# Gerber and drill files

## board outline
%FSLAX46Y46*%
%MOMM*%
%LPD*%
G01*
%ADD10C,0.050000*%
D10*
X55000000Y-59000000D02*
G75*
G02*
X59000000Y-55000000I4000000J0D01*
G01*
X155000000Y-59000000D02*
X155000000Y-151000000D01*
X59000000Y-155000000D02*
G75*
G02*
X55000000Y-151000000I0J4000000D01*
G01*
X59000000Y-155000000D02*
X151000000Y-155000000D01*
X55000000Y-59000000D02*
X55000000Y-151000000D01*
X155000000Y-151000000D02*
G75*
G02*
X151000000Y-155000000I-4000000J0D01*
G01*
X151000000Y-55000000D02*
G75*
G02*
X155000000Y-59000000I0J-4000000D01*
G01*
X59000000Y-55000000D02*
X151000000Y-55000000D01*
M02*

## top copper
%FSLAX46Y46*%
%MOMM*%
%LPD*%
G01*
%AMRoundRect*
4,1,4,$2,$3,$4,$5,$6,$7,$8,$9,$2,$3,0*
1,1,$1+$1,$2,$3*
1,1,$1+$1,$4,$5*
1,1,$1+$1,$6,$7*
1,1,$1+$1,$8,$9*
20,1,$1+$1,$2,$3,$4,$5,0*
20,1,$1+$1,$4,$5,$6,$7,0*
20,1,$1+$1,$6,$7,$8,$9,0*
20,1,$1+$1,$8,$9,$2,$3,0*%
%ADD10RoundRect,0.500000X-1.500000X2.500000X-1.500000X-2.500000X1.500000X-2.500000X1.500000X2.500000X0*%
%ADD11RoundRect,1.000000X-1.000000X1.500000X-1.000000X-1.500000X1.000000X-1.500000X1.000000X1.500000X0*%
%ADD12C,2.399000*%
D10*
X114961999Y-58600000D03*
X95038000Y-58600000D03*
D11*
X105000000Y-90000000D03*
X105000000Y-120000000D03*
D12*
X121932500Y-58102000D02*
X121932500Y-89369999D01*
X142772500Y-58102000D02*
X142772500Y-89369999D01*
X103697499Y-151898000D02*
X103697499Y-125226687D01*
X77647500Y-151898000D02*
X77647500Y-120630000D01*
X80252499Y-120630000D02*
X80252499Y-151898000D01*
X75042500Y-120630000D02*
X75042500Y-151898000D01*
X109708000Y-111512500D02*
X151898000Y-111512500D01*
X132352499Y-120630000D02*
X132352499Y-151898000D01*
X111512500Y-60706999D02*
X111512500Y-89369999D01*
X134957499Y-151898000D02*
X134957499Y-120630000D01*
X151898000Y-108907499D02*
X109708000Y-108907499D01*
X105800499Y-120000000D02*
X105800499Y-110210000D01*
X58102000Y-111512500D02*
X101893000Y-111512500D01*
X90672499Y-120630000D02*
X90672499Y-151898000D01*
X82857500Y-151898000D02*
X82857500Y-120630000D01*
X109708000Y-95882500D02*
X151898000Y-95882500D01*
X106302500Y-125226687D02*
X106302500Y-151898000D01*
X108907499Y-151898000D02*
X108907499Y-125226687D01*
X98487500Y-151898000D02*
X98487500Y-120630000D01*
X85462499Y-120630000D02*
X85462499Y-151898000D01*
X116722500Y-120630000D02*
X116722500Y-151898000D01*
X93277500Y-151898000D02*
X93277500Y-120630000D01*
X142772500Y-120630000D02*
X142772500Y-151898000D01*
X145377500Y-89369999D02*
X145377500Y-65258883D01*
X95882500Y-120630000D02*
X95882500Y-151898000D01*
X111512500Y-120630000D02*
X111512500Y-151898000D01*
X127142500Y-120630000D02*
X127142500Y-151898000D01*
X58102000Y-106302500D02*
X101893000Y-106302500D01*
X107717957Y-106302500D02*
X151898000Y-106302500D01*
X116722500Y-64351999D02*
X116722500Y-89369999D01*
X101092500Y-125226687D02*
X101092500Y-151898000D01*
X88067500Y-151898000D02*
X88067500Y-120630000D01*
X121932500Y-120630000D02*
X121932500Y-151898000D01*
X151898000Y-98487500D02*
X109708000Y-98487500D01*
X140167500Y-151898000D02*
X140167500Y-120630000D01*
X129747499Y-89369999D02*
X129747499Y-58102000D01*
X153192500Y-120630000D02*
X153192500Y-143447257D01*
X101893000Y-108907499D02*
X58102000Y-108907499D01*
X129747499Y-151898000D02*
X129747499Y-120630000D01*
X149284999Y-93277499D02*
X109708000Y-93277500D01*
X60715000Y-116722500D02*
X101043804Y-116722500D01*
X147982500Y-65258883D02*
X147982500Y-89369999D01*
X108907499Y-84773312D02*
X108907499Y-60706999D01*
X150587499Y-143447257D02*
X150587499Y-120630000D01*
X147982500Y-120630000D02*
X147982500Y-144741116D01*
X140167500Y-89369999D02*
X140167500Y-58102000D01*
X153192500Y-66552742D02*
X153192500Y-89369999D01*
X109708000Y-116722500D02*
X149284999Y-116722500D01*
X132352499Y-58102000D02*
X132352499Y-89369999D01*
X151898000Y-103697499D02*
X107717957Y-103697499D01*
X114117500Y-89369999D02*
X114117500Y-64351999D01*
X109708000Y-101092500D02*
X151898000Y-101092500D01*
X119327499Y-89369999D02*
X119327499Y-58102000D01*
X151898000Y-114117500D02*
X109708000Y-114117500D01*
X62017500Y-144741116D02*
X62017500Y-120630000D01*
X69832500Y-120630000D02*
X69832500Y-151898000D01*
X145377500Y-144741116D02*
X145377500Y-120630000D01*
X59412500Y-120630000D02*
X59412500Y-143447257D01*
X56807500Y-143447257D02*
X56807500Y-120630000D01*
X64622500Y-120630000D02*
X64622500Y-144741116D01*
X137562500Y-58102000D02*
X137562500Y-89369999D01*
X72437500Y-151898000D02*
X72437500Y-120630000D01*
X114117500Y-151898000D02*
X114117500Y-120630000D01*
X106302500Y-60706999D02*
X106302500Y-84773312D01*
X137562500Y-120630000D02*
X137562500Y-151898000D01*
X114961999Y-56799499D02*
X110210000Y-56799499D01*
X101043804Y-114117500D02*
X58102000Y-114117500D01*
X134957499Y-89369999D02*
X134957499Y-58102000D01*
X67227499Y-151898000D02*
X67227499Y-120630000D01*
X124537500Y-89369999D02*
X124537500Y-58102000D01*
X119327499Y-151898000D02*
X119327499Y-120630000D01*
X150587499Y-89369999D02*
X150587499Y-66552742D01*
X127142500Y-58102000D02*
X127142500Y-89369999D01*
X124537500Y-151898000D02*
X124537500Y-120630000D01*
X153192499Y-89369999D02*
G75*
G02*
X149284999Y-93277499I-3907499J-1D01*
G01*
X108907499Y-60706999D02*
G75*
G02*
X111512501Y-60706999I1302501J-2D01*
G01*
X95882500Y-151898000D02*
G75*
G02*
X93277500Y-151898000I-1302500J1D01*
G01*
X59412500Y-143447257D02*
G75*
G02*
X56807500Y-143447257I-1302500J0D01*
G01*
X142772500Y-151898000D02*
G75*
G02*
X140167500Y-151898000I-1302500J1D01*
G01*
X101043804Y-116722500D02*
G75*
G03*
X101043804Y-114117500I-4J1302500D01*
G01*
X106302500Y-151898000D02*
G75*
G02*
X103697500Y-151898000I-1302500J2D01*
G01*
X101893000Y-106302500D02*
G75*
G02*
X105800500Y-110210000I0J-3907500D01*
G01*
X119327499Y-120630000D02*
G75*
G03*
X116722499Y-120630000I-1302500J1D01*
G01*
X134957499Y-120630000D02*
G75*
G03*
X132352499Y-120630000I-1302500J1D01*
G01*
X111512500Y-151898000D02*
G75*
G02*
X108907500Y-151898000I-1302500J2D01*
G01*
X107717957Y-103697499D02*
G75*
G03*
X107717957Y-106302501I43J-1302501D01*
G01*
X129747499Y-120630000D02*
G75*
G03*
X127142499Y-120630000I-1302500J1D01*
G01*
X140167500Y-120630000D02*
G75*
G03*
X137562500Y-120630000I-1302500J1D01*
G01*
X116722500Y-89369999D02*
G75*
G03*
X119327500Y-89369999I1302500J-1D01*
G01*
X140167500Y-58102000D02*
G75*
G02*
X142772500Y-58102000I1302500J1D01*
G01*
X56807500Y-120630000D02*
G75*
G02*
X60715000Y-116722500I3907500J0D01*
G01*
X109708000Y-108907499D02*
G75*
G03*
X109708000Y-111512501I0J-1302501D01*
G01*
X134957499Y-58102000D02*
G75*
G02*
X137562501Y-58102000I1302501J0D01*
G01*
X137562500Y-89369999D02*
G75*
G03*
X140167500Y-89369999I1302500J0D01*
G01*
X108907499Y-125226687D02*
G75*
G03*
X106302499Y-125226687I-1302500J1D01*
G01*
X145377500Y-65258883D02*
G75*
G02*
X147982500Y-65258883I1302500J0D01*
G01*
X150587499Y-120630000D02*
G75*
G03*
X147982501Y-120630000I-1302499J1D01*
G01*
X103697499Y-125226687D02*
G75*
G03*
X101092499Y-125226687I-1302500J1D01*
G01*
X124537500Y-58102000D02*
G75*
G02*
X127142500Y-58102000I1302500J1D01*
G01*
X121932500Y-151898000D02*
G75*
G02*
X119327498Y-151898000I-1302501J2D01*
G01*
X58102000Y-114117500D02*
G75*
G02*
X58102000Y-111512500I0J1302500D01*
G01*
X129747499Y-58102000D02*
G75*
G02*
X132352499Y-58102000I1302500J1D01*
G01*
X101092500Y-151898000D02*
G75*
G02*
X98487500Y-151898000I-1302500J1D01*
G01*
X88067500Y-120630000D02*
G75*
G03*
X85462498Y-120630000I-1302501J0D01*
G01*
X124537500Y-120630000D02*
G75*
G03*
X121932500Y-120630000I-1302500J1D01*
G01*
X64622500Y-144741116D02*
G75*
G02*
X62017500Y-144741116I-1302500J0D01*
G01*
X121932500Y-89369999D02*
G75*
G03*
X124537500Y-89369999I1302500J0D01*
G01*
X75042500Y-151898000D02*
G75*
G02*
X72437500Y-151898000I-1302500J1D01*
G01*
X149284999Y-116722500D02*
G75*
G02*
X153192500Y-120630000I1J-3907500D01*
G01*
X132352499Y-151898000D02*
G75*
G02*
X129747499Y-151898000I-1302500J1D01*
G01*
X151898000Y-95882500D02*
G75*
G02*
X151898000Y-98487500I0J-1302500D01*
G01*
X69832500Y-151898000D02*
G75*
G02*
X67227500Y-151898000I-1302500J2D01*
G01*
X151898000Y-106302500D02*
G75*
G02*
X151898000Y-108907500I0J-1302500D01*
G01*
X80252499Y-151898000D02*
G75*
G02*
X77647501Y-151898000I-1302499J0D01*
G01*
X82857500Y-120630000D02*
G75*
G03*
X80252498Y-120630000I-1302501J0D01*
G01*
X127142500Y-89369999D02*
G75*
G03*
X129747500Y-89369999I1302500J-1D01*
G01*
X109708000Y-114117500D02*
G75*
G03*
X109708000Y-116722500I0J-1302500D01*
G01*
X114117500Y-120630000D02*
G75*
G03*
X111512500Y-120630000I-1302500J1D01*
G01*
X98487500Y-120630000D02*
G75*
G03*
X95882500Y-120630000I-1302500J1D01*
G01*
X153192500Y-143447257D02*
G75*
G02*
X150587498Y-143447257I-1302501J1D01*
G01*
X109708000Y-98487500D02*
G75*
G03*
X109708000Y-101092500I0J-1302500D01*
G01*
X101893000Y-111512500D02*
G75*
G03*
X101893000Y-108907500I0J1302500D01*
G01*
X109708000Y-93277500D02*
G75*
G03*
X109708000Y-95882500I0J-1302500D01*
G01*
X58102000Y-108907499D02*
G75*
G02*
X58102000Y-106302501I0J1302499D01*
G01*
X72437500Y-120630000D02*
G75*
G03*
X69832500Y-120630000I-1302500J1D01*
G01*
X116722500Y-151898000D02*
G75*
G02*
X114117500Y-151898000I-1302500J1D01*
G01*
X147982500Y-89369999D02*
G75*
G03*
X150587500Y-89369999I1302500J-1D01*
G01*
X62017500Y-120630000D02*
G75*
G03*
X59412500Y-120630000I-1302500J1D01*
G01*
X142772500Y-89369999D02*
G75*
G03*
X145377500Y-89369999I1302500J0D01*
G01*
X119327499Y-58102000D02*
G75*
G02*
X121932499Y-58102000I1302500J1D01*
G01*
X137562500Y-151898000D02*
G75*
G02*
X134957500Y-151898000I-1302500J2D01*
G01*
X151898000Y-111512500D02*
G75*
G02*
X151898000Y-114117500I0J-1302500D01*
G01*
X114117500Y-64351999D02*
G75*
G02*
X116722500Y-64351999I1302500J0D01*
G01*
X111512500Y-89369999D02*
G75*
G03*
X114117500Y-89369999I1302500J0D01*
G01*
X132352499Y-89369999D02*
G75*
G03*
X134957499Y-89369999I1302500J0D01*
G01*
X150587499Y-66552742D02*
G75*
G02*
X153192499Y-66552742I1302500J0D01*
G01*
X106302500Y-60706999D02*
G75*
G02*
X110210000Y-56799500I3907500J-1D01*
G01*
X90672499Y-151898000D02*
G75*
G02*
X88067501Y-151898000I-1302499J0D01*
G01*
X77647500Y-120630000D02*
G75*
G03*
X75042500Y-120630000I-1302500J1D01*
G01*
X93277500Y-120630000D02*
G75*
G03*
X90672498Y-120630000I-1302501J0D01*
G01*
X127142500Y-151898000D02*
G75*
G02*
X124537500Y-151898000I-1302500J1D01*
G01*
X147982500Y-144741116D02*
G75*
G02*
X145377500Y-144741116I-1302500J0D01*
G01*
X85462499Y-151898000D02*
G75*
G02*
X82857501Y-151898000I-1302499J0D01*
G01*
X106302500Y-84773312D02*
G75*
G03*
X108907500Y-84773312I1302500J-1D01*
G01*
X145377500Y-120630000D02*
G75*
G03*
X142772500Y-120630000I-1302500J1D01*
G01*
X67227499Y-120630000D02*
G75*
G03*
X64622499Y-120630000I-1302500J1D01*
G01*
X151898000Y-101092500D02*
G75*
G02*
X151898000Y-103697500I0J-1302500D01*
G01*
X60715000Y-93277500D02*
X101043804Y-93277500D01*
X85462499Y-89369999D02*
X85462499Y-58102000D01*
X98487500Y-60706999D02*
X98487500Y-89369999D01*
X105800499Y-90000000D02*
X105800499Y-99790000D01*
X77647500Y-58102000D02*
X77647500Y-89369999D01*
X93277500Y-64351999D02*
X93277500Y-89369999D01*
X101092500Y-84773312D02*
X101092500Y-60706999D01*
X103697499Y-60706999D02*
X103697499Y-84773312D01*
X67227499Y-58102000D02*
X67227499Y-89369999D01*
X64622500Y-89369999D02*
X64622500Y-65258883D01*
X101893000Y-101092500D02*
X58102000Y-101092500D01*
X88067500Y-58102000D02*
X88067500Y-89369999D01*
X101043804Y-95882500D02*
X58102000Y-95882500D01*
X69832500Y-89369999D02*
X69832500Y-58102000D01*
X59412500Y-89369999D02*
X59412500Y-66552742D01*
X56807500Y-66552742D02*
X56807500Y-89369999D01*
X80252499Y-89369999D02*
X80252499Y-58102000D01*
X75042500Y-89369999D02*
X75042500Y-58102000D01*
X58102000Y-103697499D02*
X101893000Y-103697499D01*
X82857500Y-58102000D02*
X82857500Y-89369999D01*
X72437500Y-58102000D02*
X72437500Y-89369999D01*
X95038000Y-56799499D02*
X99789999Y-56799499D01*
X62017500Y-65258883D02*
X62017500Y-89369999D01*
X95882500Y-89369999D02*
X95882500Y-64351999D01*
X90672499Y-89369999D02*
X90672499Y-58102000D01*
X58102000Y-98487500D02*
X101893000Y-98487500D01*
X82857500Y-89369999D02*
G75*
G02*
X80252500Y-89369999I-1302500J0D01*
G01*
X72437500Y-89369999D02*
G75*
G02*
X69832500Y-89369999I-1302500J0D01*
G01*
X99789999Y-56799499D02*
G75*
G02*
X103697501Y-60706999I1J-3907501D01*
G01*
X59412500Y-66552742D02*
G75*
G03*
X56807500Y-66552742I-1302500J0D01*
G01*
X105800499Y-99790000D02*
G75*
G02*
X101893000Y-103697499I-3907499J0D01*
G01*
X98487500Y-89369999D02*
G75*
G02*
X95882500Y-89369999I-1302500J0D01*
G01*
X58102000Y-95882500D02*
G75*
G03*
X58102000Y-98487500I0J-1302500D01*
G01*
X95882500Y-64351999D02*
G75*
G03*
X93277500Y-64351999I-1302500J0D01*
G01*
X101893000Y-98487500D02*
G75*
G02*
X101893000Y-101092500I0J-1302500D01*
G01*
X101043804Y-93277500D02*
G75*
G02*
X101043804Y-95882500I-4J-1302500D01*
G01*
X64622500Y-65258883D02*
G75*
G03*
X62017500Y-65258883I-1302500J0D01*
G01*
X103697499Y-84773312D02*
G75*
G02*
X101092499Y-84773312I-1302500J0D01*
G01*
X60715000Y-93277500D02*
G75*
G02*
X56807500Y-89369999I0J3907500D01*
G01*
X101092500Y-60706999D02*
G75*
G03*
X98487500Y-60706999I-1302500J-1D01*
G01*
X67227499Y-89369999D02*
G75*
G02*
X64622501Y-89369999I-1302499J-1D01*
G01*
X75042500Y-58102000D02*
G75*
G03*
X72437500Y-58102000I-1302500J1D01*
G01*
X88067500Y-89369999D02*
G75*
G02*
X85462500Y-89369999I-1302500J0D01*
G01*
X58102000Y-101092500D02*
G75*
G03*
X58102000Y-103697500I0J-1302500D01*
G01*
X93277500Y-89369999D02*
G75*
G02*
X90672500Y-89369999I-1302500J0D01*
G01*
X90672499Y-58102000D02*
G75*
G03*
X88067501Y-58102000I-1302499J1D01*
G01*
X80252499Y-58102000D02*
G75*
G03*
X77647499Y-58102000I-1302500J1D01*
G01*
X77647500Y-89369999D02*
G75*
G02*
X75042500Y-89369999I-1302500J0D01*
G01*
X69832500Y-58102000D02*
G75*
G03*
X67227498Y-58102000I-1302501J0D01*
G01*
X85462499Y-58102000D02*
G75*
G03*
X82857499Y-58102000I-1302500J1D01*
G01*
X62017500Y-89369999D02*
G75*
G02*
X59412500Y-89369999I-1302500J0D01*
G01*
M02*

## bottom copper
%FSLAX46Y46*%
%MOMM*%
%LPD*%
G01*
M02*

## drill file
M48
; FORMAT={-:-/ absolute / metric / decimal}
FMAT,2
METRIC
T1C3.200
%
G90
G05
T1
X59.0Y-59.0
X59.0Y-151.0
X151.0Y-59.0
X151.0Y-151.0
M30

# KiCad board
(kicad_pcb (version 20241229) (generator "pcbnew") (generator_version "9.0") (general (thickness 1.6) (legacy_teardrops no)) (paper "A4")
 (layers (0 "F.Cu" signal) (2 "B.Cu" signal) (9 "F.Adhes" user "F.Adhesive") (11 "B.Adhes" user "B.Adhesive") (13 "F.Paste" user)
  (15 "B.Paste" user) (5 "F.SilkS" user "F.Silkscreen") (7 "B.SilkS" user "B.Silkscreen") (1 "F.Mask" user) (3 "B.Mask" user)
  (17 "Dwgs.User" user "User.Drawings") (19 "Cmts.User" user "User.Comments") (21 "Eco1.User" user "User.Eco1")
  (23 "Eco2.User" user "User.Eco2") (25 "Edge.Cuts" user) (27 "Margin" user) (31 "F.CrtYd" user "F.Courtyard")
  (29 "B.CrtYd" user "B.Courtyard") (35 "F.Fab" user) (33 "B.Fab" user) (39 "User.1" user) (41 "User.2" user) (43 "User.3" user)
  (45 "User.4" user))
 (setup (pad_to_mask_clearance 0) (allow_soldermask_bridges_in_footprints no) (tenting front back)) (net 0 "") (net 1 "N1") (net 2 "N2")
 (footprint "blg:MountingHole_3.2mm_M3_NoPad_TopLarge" (layer "F.Cu") (at 151 59)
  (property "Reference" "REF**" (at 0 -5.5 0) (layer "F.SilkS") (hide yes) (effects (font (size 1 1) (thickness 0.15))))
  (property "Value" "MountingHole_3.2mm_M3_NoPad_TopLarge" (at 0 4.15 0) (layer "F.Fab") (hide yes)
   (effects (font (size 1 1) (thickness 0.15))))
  (pad "" np_thru_hole circle (at 0 0) (size 7.6 7.6) (drill 3.2) (layers) (zone_connect 2)))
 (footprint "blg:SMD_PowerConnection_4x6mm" (layer "F.Cu") (at 114.961999 58.6 -90)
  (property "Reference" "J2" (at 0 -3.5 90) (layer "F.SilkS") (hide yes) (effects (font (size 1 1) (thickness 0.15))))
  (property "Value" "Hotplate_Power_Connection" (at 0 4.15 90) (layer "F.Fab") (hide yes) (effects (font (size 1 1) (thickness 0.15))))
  (pad "1" smd roundrect (at 0 0 270) (size 6 4) (layers "F.Cu" "F.Mask" "F.Paste") (roundrect_rratio 0.125) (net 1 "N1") (zone_connect 2)))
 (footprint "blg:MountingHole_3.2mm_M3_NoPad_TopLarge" (layer "F.Cu") (at 59 151)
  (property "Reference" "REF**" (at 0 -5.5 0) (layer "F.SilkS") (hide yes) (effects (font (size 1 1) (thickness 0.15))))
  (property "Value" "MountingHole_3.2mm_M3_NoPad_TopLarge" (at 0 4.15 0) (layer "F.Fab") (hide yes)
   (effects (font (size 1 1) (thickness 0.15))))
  (pad "" np_thru_hole circle (at 0 0) (size 7.6 7.6) (drill 3.2) (layers) (zone_connect 2)))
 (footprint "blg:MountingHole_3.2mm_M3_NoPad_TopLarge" (layer "F.Cu") (at 151 151)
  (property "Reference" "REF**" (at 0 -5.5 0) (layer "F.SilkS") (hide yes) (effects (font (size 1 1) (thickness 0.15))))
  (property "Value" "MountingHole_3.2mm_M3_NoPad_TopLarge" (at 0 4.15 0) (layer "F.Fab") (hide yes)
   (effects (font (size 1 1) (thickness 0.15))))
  (pad "" np_thru_hole circle (at 0 0) (size 7.6 7.6) (drill 3.2) (layers) (zone_connect 2)))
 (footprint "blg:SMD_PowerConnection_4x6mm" (layer "F.Cu") (at 95.038 58.6 -90)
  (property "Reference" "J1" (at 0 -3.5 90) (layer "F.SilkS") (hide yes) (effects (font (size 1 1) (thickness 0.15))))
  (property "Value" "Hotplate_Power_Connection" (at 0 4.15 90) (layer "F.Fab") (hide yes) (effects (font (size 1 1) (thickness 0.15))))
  (pad "1" smd roundrect (at 0 0 270) (size 6 4) (layers "F.Cu" "F.Mask" "F.Paste") (roundrect_rratio 0.125) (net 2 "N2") (zone_connect 2)))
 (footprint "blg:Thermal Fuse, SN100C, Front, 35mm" (layer "F.Cu") (at 105 105 -90)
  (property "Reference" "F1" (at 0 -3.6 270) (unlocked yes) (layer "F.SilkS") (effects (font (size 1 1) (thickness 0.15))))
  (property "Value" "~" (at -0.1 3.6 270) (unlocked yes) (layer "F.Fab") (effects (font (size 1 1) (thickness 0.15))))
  (pad "1" smd roundrect (at -15 0 270) (size 5 4) (layers "F.Cu" "F.Mask") (roundrect_rratio 0.25) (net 2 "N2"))
  (pad "2" smd roundrect (at 15 0 270) (size 5 4) (layers "F.Cu" "F.Mask") (roundrect_rratio 0.25) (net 1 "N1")))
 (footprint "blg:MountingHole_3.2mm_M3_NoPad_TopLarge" (layer "F.Cu") (at 59 59)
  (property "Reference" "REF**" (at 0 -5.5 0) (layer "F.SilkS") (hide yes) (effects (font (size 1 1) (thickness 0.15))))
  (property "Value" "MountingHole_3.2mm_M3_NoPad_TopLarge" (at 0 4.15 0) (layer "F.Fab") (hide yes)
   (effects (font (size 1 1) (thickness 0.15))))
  (pad "" np_thru_hole circle (at 0 0) (size 7.6 7.6) (drill 3.2) (layers) (zone_connect 2)))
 (gr_arc (start 55 59) (mid 56.171573 56.171573) (end 59 55) (stroke (width 0.05) (type solid)) (layer "Edge.Cuts"))
 (gr_line (start 155 59) (end 155 151) (stroke (width 0.05) (type default)) (layer "Edge.Cuts"))
 (gr_arc (start 59 155) (mid 56.171573 153.828427) (end 55 151) (stroke (width 0.05) (type solid)) (layer "Edge.Cuts"))
 (gr_line (start 59 155) (end 151 155) (stroke (width 0.05) (type default)) (layer "Edge.Cuts"))
 (gr_line (start 55 59) (end 55 151) (stroke (width 0.05) (type default)) (layer "Edge.Cuts"))
 (gr_arc (start 155 151) (mid 153.828427 153.828427) (end 151 155) (stroke (width 0.05) (type solid)) (layer "Edge.Cuts"))
 (gr_arc (start 151 55) (mid 153.828427 56.171573) (end 155 59) (stroke (width 0.05) (type solid)) (layer "Edge.Cuts"))
 (gr_line (start 59 55) (end 151 55) (stroke (width 0.05) (type default)) (layer "Edge.Cuts"))
 (segment (start 121.9325 58.102) (end 121.9325 89.369999) (width 2.399) (layer "F.Cu") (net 1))
 (segment (start 142.7725 58.102) (end 142.7725 89.369999) (width 2.399) (layer "F.Cu") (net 1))
 (segment (start 103.697499 151.898) (end 103.697499 125.226687) (width 2.399) (layer "F.Cu") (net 1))
 (segment (start 77.6475 151.898) (end 77.6475 120.63) (width 2.399) (layer "F.Cu") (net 1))
 (segment (start 80.252499 120.63) (end 80.252499 151.898) (width 2.399) (layer "F.Cu") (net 1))
 (segment (start 75.0425 120.63) (end 75.0425 151.898) (width 2.399) (layer "F.Cu") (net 1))
 (segment (start 109.708 111.5125) (end 151.898 111.5125) (width 2.399) (layer "F.Cu") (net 1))
 (segment (start 132.352499 120.63) (end 132.352499 151.898) (width 2.399) (layer "F.Cu") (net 1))
 (segment (start 111.5125 60.706999) (end 111.5125 89.369999) (width 2.399) (layer "F.Cu") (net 1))
 (segment (start 134.957499 151.898) (end 134.957499 120.63) (width 2.399) (layer "F.Cu") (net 1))
 (segment (start 151.898 108.907499) (end 109.708 108.907499) (width 2.399) (layer "F.Cu") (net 1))
 (segment (start 105.800499 120) (end 105.800499 110.21) (width 2.399) (layer "F.Cu") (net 1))
 (segment (start 58.102 111.5125) (end 101.893 111.5125) (width 2.399) (layer "F.Cu") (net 1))
 (segment (start 90.672499 120.63) (end 90.672499 151.898) (width 2.399) (layer "F.Cu") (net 1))
 (segment (start 82.8575 151.898) (end 82.8575 120.63) (width 2.399) (layer "F.Cu") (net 1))
 (segment (start 109.708 95.8825) (end 151.898 95.8825) (width 2.399) (layer "F.Cu") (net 1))
 (segment (start 106.3025 125.226687) (end 106.3025 151.898) (width 2.399) (layer "F.Cu") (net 1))
 (segment (start 108.907499 151.898) (end 108.907499 125.226687) (width 2.399) (layer "F.Cu") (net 1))
 (segment (start 98.4875 151.898) (end 98.4875 120.63) (width 2.399) (layer "F.Cu") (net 1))
 (segment (start 85.462499 120.63) (end 85.462499 151.898) (width 2.399) (layer "F.Cu") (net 1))
 (segment (start 116.7225 120.63) (end 116.7225 151.898) (width 2.399) (layer "F.Cu") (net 1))
 (segment (start 93.2775 151.898) (end 93.2775 120.63) (width 2.399) (layer "F.Cu") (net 1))
 (segment (start 142.7725 120.63) (end 142.7725 151.898) (width 2.399) (layer "F.Cu") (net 1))
 (segment (start 145.3775 89.369999) (end 145.3775 65.258883) (width 2.399) (layer "F.Cu") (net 1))
 (segment (start 95.8825 120.63) (end 95.8825 151.898) (width 2.399) (layer "F.Cu") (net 1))
 (segment (start 111.5125 120.63) (end 111.5125 151.898) (width 2.399) (layer "F.Cu") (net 1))
 (segment (start 127.1425 120.63) (end 127.1425 151.898) (width 2.399) (layer "F.Cu") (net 1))
 (segment (start 58.102 106.3025) (end 101.893 106.3025) (width 2.399) (layer "F.Cu") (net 1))
 (segment (start 107.717957 106.3025) (end 151.898 106.3025) (width 2.399) (layer "F.Cu") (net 1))
 (segment (start 116.7225 64.351999) (end 116.7225 89.369999) (width 2.399) (layer "F.Cu") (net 1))
 (segment (start 101.0925 125.226687) (end 101.0925 151.898) (width 2.399) (layer "F.Cu") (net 1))
 (segment (start 88.0675 151.898) (end 88.0675 120.63) (width 2.399) (layer "F.Cu") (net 1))
 (segment (start 121.9325 120.63) (end 121.9325 151.898) (width 2.399) (layer "F.Cu") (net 1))
 (segment (start 151.898 98.4875) (end 109.708 98.4875) (width 2.399) (layer "F.Cu") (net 1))
 (segment (start 140.1675 151.898) (end 140.1675 120.63) (width 2.399) (layer "F.Cu") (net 1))
 (segment (start 129.747499 89.369999) (end 129.747499 58.102) (width 2.399) (layer "F.Cu") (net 1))
 (segment (start 153.1925 120.63) (end 153.1925 143.447257) (width 2.399) (layer "F.Cu") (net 1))
 (segment (start 101.893 108.907499) (end 58.102 108.907499) (width 2.399) (layer "F.Cu") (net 1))
 (segment (start 129.747499 151.898) (end 129.747499 120.63) (width 2.399) (layer "F.Cu") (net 1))
 (segment (start 149.284999 93.277499) (end 109.708 93.2775) (width 2.399) (layer "F.Cu") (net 1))
 (segment (start 60.715 116.7225) (end 101.043804 116.7225) (width 2.399) (layer "F.Cu") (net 1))
 (segment (start 147.9825 65.258883) (end 147.9825 89.369999) (width 2.399) (layer "F.Cu") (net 1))
 (segment (start 108.907499 84.773312) (end 108.907499 60.706999) (width 2.399) (layer "F.Cu") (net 1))
 (segment (start 150.587499 143.447257) (end 150.587499 120.63) (width 2.399) (layer "F.Cu") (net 1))
 (segment (start 147.9825 120.63) (end 147.9825 144.741116) (width 2.399) (layer "F.Cu") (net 1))
 (segment (start 140.1675 89.369999) (end 140.1675 58.102) (width 2.399) (layer "F.Cu") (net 1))
 (segment (start 153.1925 66.552742) (end 153.1925 89.369999) (width 2.399) (layer "F.Cu") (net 1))
 (segment (start 109.708 116.7225) (end 149.284999 116.7225) (width 2.399) (layer "F.Cu") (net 1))
 (segment (start 132.352499 58.102) (end 132.352499 89.369999) (width 2.399) (layer "F.Cu") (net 1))
 (segment (start 151.898 103.697499) (end 107.717957 103.697499) (width 2.399) (layer "F.Cu") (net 1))
 (segment (start 114.1175 89.369999) (end 114.1175 64.351999) (width 2.399) (layer "F.Cu") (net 1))
 (segment (start 109.708 101.0925) (end 151.898 101.0925) (width 2.399) (layer "F.Cu") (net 1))
 (segment (start 119.327499 89.369999) (end 119.327499 58.102) (width 2.399) (layer "F.Cu") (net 1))
 (segment (start 151.898 114.1175) (end 109.708 114.1175) (width 2.399) (layer "F.Cu") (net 1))
 (segment (start 62.0175 144.741116) (end 62.0175 120.63) (width 2.399) (layer "F.Cu") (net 1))
 (segment (start 69.8325 120.63) (end 69.8325 151.898) (width 2.399) (layer "F.Cu") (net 1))
 (segment (start 145.3775 144.741116) (end 145.3775 120.63) (width 2.399) (layer "F.Cu") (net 1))
 (segment (start 59.4125 120.63) (end 59.4125 143.447257) (width 2.399) (layer "F.Cu") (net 1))
 (segment (start 56.8075 143.447257) (end 56.8075 120.63) (width 2.399) (layer "F.Cu") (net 1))
 (segment (start 64.6225 120.63) (end 64.6225 144.741116) (width 2.399) (layer "F.Cu") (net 1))
 (segment (start 137.5625 58.102) (end 137.5625 89.369999) (width 2.399) (layer "F.Cu") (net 1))
 (segment (start 72.4375 151.898) (end 72.4375 120.63) (width 2.399) (layer "F.Cu") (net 1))
 (segment (start 114.1175 151.898) (end 114.1175 120.63) (width 2.399) (layer "F.Cu") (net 1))
 (segment (start 106.3025 60.706999) (end 106.3025 84.773312) (width 2.399) (layer "F.Cu") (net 1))
 (segment (start 137.5625 120.63) (end 137.5625 151.898) (width 2.399) (layer "F.Cu") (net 1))
 (segment (start 114.961999 56.799499) (end 110.21 56.799499) (width 2.399) (layer "F.Cu") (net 1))
 (segment (start 101.043804 114.1175) (end 58.102 114.1175) (width 2.399) (layer "F.Cu") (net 1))
 (segment (start 134.957499 89.369999) (end 134.957499 58.102) (width 2.399) (layer "F.Cu") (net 1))
 (segment (start 67.227499 151.898) (end 67.227499 120.63) (width 2.399) (layer "F.Cu") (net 1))
 (segment (start 124.5375 89.369999) (end 124.5375 58.102) (width 2.399) (layer "F.Cu") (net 1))
 (segment (start 119.327499 151.898) (end 119.327499 120.63) (width 2.399) (layer "F.Cu") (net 1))
 (segment (start 150.587499 89.369999) (end 150.587499 66.552742) (width 2.399) (layer "F.Cu") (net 1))
 (segment (start 127.1425 58.102) (end 127.1425 89.369999) (width 2.399) (layer "F.Cu") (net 1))
 (segment (start 124.5375 151.898) (end 124.5375 120.63) (width 2.399) (layer "F.Cu") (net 1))
 (arc (start 153.192499 89.369999) (mid 152.048019 92.133019) (end 149.284999 93.277499) (width 2.399) (layer "F.Cu") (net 1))
 (arc (start 108.907499 60.706999) (mid 110.21 59.4045) (end 111.5125 60.706999) (width 2.399) (layer "F.Cu") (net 1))
 (arc (start 95.8825 151.898) (mid 94.58 153.200499) (end 93.2775 151.898) (width 2.399) (layer "F.Cu") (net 1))
 (arc (start 59.4125 143.447257) (mid 58.109999 144.749757) (end 56.8075 143.447257) (width 2.399) (layer "F.Cu") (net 1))
 (arc (start 142.7725 151.898) (mid 141.469999 153.200499) (end 140.1675 151.898) (width 2.399) (layer "F.Cu") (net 1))
 (arc (start 101.043804 116.7225) (mid 102.346304 115.42) (end 101.043804 114.1175) (width 2.399) (layer "F.Cu") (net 1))
 (arc (start 106.3025 151.898) (mid 105 153.200499) (end 103.697499 151.898) (width 2.399) (layer "F.Cu") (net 1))
 (arc (start 101.893 106.3025) (mid 104.656019 107.44698) (end 105.800499 110.21) (width 2.399) (layer "F.Cu") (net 1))
 (arc (start 119.327499 120.63) (mid 118.024999 119.327499) (end 116.7225 120.63) (width 2.399) (layer "F.Cu") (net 1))
 (arc (start 134.957499 120.63) (mid 133.655 119.327499) (end 132.352499 120.63) (width 2.399) (layer "F.Cu") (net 1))
 (arc (start 111.5125 151.898) (mid 110.21 153.200499) (end 108.907499 151.898) (width 2.399) (layer "F.Cu") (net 1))
 (arc (start 107.717957 103.697499) (mid 106.415457 105) (end 107.717957 106.3025) (width 2.399) (layer "F.Cu") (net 1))
 (arc (start 129.747499 120.63) (mid 128.445 119.327499) (end 127.1425 120.63) (width 2.399) (layer "F.Cu") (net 1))
 (arc (start 140.1675 120.63) (mid 138.864999 119.327499) (end 137.5625 120.63) (width 2.399) (layer "F.Cu") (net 1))
 (arc (start 116.7225 89.369999) (mid 118.024999 90.672499) (end 119.327499 89.369999) (width 2.399) (layer "F.Cu") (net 1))
 (arc (start 140.1675 58.102) (mid 141.469999 56.799499) (end 142.7725 58.102) (width 2.399) (layer "F.Cu") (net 1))
 (arc (start 56.8075 120.63) (mid 57.95198 117.86698) (end 60.715 116.7225) (width 2.399) (layer "F.Cu") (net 1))
 (arc (start 109.708 108.907499) (mid 108.4055 110.21) (end 109.708 111.5125) (width 2.399) (layer "F.Cu") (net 1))
 (arc (start 134.957499 58.102) (mid 136.26 56.799499) (end 137.5625 58.102) (width 2.399) (layer "F.Cu") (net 1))
 (arc (start 137.5625 89.369999) (mid 138.864999 90.672499) (end 140.1675 89.369999) (width 2.399) (layer "F.Cu") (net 1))
 (arc (start 108.907499 125.226687) (mid 107.604999 123.924186) (end 106.3025 125.226687) (width 2.399) (layer "F.Cu") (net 1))
 (arc (start 145.3775 65.258883) (mid 146.68 63.956383) (end 147.9825 65.258883) (width 2.399) (layer "F.Cu") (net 1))
 (arc (start 150.587499 120.63) (mid 149.285 119.327499) (end 147.9825 120.63) (width 2.399) (layer "F.Cu") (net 1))
 (arc (start 103.697499 125.226687) (mid 102.395 123.924186) (end 101.0925 125.226687) (width 2.399) (layer "F.Cu") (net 1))
 (arc (start 124.5375 58.102) (mid 125.84 56.799499) (end 127.1425 58.102) (width 2.399) (layer "F.Cu") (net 1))
 (arc (start 121.9325 151.898) (mid 120.63 153.200499) (end 119.327499 151.898) (width 2.399) (layer "F.Cu") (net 1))
 (arc (start 58.102 114.1175) (mid 56.799499 112.815) (end 58.102 111.5125) (width 2.399) (layer "F.Cu") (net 1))
 (arc (start 129.747499 58.102) (mid 131.05 56.799499) (end 132.352499 58.102) (width 2.399) (layer "F.Cu") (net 1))
 (arc (start 101.0925 151.898) (mid 99.789999 153.200499) (end 98.4875 151.898) (width 2.399) (layer "F.Cu") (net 1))
 (arc (start 88.0675 120.63) (mid 86.765 119.327499) (end 85.462499 120.63) (width 2.399) (layer "F.Cu") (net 1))
 (arc (start 124.5375 120.63) (mid 123.235 119.327499) (end 121.9325 120.63) (width 2.399) (layer "F.Cu") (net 1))
 (arc (start 64.6225 144.741116) (mid 63.32 146.043616) (end 62.0175 144.741116) (width 2.399) (layer "F.Cu") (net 1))
 (arc (start 121.9325 89.369999) (mid 123.235 90.672499) (end 124.5375 89.369999) (width 2.399) (layer "F.Cu") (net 1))
 (arc (start 75.0425 151.898) (mid 73.74 153.200499) (end 72.4375 151.898) (width 2.399) (layer "F.Cu") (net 1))
 (arc (start 149.284999 116.7225) (mid 152.048019 117.86698) (end 153.192499 120.63) (width 2.399) (layer "F.Cu") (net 1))
 (arc (start 132.352499 151.898) (mid 131.05 153.200499) (end 129.747499 151.898) (width 2.399) (layer "F.Cu") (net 1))
 (arc (start 151.898 95.8825) (mid 153.200499 97.184999) (end 151.898 98.4875) (width 2.399) (layer "F.Cu") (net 1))
 (arc (start 69.8325 151.898) (mid 68.529999 153.200499) (end 67.227499 151.898) (width 2.399) (layer "F.Cu") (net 1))
 (arc (start 151.898 106.3025) (mid 153.200499 107.604999) (end 151.898 108.907499) (width 2.399) (layer "F.Cu") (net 1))
 (arc (start 80.252499 151.898) (mid 78.949999 153.200499) (end 77.6475 151.898) (width 2.399) (layer "F.Cu") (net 1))
 (arc (start 82.8575 120.63) (mid 81.555 119.327499) (end 80.252499 120.63) (width 2.399) (layer "F.Cu") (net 1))
 (arc (start 127.1425 89.369999) (mid 128.445 90.672499) (end 129.747499 89.369999) (width 2.399) (layer "F.Cu") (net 1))
 (arc (start 109.708 114.1175) (mid 108.4055 115.42) (end 109.708 116.7225) (width 2.399) (layer "F.Cu") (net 1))
 (arc (start 114.1175 120.63) (mid 112.815 119.327499) (end 111.5125 120.63) (width 2.399) (layer "F.Cu") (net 1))
 (arc (start 98.4875 120.63) (mid 97.184999 119.327499) (end 95.8825 120.63) (width 2.399) (layer "F.Cu") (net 1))
 (arc (start 153.1925 143.447257) (mid 151.89 144.749757) (end 150.587499 143.447257) (width 2.399) (layer "F.Cu") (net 1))
 (arc (start 109.708 98.4875) (mid 108.4055 99.789999) (end 109.708 101.0925) (width 2.399) (layer "F.Cu") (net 1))
 (arc (start 101.893 111.5125) (mid 103.1955 110.21) (end 101.893 108.907499) (width 2.399) (layer "F.Cu") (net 1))
 (arc (start 109.708 93.2775) (mid 108.4055 94.58) (end 109.708 95.8825) (width 2.399) (layer "F.Cu") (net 1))
 (arc (start 58.102 108.907499) (mid 56.799499 107.604999) (end 58.102 106.3025) (width 2.399) (layer "F.Cu") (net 1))
 (arc (start 72.4375 120.63) (mid 71.134999 119.327499) (end 69.8325 120.63) (width 2.399) (layer "F.Cu") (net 1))
 (arc (start 116.7225 151.898) (mid 115.42 153.200499) (end 114.1175 151.898) (width 2.399) (layer "F.Cu") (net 1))
 (arc (start 147.9825 89.369999) (mid 149.285 90.672499) (end 150.587499 89.369999) (width 2.399) (layer "F.Cu") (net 1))
 (arc (start 62.0175 120.63) (mid 60.715 119.327499) (end 59.4125 120.63) (width 2.399) (layer "F.Cu") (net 1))
 (arc (start 142.7725 89.369999) (mid 144.075 90.672499) (end 145.3775 89.369999) (width 2.399) (layer "F.Cu") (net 1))
 (arc (start 119.327499 58.102) (mid 120.63 56.799499) (end 121.9325 58.102) (width 2.399) (layer "F.Cu") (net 1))
 (arc (start 137.5625 151.898) (mid 136.26 153.200499) (end 134.957499 151.898) (width 2.399) (layer "F.Cu") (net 1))
 (arc (start 151.898 111.5125) (mid 153.200499 112.815) (end 151.898 114.1175) (width 2.399) (layer "F.Cu") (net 1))
 (arc (start 114.1175 64.351999) (mid 115.42 63.049499) (end 116.7225 64.351999) (width 2.399) (layer "F.Cu") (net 1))
 (arc (start 111.5125 89.369999) (mid 112.815 90.672499) (end 114.1175 89.369999) (width 2.399) (layer "F.Cu") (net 1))
 (arc (start 132.352499 89.369999) (mid 133.655 90.672499) (end 134.957499 89.369999) (width 2.399) (layer "F.Cu") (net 1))
 (arc (start 150.587499 66.552742) (mid 151.89 65.250242) (end 153.1925 66.552742) (width 2.399) (layer "F.Cu") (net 1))
 (arc (start 106.3025 60.706999) (mid 107.44698 57.94398) (end 110.21 56.799499) (width 2.399) (layer "F.Cu") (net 1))
 (arc (start 90.672499 151.898) (mid 89.369999 153.200499) (end 88.0675 151.898) (width 2.399) (layer "F.Cu") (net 1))
 (arc (start 77.6475 120.63) (mid 76.345 119.327499) (end 75.0425 120.63) (width 2.399) (layer "F.Cu") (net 1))
 (arc (start 93.2775 120.63) (mid 91.975 119.327499) (end 90.672499 120.63) (width 2.399) (layer "F.Cu") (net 1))
 (arc (start 127.1425 151.898) (mid 125.84 153.200499) (end 124.5375 151.898) (width 2.399) (layer "F.Cu") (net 1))
 (arc (start 147.9825 144.741116) (mid 146.68 146.043616) (end 145.3775 144.741116) (width 2.399) (layer "F.Cu") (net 1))
 (arc (start 85.462499 151.898) (mid 84.16 153.200499) (end 82.8575 151.898) (width 2.399) (layer "F.Cu") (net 1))
 (arc (start 106.3025 84.773312) (mid 107.604999 86.075812) (end 108.907499 84.773312) (width 2.399) (layer "F.Cu") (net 1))
 (arc (start 145.3775 120.63) (mid 144.075 119.327499) (end 142.7725 120.63) (width 2.399) (layer "F.Cu") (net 1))
 (arc (start 67.227499 120.63) (mid 65.925 119.327499) (end 64.6225 120.63) (width 2.399) (layer "F.Cu") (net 1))
 (arc (start 151.898 101.0925) (mid 153.200499 102.395) (end 151.898 103.697499) (width 2.399) (layer "F.Cu") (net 1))
 (segment (start 60.715 93.2775) (end 101.043804 93.2775) (width 2.399) (layer "F.Cu") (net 2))
 (segment (start 85.462499 89.369999) (end 85.462499 58.102) (width 2.399) (layer "F.Cu") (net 2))
 (segment (start 98.4875 60.706999) (end 98.4875 89.369999) (width 2.399) (layer "F.Cu") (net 2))
 (segment (start 105.800499 90) (end 105.800499 99.79) (width 2.399) (layer "F.Cu") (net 2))
 (segment (start 77.6475 58.102) (end 77.6475 89.369999) (width 2.399) (layer "F.Cu") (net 2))
 (segment (start 93.2775 64.351999) (end 93.2775 89.369999) (width 2.399) (layer "F.Cu") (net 2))
 (segment (start 101.0925 84.773312) (end 101.0925 60.706999) (width 2.399) (layer "F.Cu") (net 2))
 (segment (start 103.697499 60.706999) (end 103.697499 84.773312) (width 2.399) (layer "F.Cu") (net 2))
 (segment (start 67.227499 58.102) (end 67.227499 89.369999) (width 2.399) (layer "F.Cu") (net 2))
 (segment (start 64.6225 89.369999) (end 64.6225 65.258883) (width 2.399) (layer "F.Cu") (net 2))
 (segment (start 101.893 101.0925) (end 58.102 101.0925) (width 2.399) (layer "F.Cu") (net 2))
 (segment (start 88.0675 58.102) (end 88.0675 89.369999) (width 2.399) (layer "F.Cu") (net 2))
 (segment (start 101.043804 95.8825) (end 58.102 95.8825) (width 2.399) (layer "F.Cu") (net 2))
 (segment (start 69.8325 89.369999) (end 69.8325 58.102) (width 2.399) (layer "F.Cu") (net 2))
 (segment (start 59.4125 89.369999) (end 59.4125 66.552742) (width 2.399) (layer "F.Cu") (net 2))
 (segment (start 56.8075 66.552742) (end 56.8075 89.369999) (width 2.399) (layer "F.Cu") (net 2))
 (segment (start 80.252499 89.369999) (end 80.252499 58.102) (width 2.399) (layer "F.Cu") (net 2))
 (segment (start 75.0425 89.369999) (end 75.0425 58.102) (width 2.399) (layer "F.Cu") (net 2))
 (segment (start 58.102 103.697499) (end 101.893 103.697499) (width 2.399) (layer "F.Cu") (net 2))
 (segment (start 82.8575 58.102) (end 82.8575 89.369999) (width 2.399) (layer "F.Cu") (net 2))
 (segment (start 72.4375 58.102) (end 72.4375 89.369999) (width 2.399) (layer "F.Cu") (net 2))
 (segment (start 95.038 56.799499) (end 99.789999 56.799499) (width 2.399) (layer "F.Cu") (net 2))
 (segment (start 62.0175 65.258883) (end 62.0175 89.369999) (width 2.399) (layer "F.Cu") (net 2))
 (segment (start 95.8825 89.369999) (end 95.8825 64.351999) (width 2.399) (layer "F.Cu") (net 2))
 (segment (start 90.672499 89.369999) (end 90.672499 58.102) (width 2.399) (layer "F.Cu") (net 2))
 (segment (start 58.102 98.4875) (end 101.893 98.4875) (width 2.399) (layer "F.Cu") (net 2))
 (arc (start 82.8575 89.369999) (mid 81.555 90.672499) (end 80.252499 89.369999) (width 2.399) (layer "F.Cu") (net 2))
 (arc (start 72.4375 89.369999) (mid 71.134999 90.672499) (end 69.8325 89.369999) (width 2.399) (layer "F.Cu") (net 2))
 (arc (start 99.789999 56.799499) (mid 102.553019 57.94398) (end 103.697499 60.706999) (width 2.399) (layer "F.Cu") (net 2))
 (arc (start 59.4125 66.552742) (mid 58.109999 65.250242) (end 56.8075 66.552742) (width 2.399) (layer "F.Cu") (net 2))
 (arc (start 105.800499 99.79) (mid 104.656019 102.553019) (end 101.893 103.697499) (width 2.399) (layer "F.Cu") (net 2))
 (arc (start 98.4875 89.369999) (mid 97.184999 90.672499) (end 95.8825 89.369999) (width 2.399) (layer "F.Cu") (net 2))
 (arc (start 58.102 95.8825) (mid 56.799499 97.184999) (end 58.102 98.4875) (width 2.399) (layer "F.Cu") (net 2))
 (arc (start 95.8825 64.351999) (mid 94.58 63.049499) (end 93.2775 64.351999) (width 2.399) (layer "F.Cu") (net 2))
 (arc (start 101.893 98.4875) (mid 103.1955 99.789999) (end 101.893 101.0925) (width 2.399) (layer "F.Cu") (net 2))
 (arc (start 101.043804 93.2775) (mid 102.346304 94.58) (end 101.043804 95.8825) (width 2.399) (layer "F.Cu") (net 2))
 (arc (start 64.6225 65.258883) (mid 63.32 63.956383) (end 62.0175 65.258883) (width 2.399) (layer "F.Cu") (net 2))
 (arc (start 103.697499 84.773312) (mid 102.395 86.075812) (end 101.0925 84.773312) (width 2.399) (layer "F.Cu") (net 2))
 (arc (start 60.715 93.2775) (mid 57.95198 92.133019) (end 56.8075 89.369999) (width 2.399) (layer "F.Cu") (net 2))
 (arc (start 101.0925 60.706999) (mid 99.789999 59.4045) (end 98.4875 60.706999) (width 2.399) (layer "F.Cu") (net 2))
 (arc (start 67.227499 89.369999) (mid 65.925 90.672499) (end 64.6225 89.369999) (width 2.399) (layer "F.Cu") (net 2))
 (arc (start 75.0425 58.102) (mid 73.74 56.799499) (end 72.4375 58.102) (width 2.399) (layer "F.Cu") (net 2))
 (arc (start 88.0675 89.369999) (mid 86.765 90.672499) (end 85.462499 89.369999) (width 2.399) (layer "F.Cu") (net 2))
 (arc (start 58.102 101.0925) (mid 56.799499 102.395) (end 58.102 103.697499) (width 2.399) (layer "F.Cu") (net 2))
 (arc (start 93.2775 89.369999) (mid 91.975 90.672499) (end 90.672499 89.369999) (width 2.399) (layer "F.Cu") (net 2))
 (arc (start 90.672499 58.102) (mid 89.369999 56.799499) (end 88.0675 58.102) (width 2.399) (layer "F.Cu") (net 2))
 (arc (start 80.252499 58.102) (mid 78.949999 56.799499) (end 77.6475 58.102) (width 2.399) (layer "F.Cu") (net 2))
 (arc (start 77.6475 89.369999) (mid 76.345 90.672499) (end 75.0425 89.369999) (width 2.399) (layer "F.Cu") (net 2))
 (arc (start 69.8325 58.102) (mid 68.529999 56.799499) (end 67.227499 58.102) (width 2.399) (layer "F.Cu") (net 2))
 (arc (start 85.462499 58.102) (mid 84.16 56.799499) (end 82.8575 58.102) (width 2.399) (layer "F.Cu") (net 2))
 (arc (start 62.0175 89.369999) (mid 60.715 90.672499) (end 59.4125 89.369999) (width 2.399) (layer "F.Cu") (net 2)))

